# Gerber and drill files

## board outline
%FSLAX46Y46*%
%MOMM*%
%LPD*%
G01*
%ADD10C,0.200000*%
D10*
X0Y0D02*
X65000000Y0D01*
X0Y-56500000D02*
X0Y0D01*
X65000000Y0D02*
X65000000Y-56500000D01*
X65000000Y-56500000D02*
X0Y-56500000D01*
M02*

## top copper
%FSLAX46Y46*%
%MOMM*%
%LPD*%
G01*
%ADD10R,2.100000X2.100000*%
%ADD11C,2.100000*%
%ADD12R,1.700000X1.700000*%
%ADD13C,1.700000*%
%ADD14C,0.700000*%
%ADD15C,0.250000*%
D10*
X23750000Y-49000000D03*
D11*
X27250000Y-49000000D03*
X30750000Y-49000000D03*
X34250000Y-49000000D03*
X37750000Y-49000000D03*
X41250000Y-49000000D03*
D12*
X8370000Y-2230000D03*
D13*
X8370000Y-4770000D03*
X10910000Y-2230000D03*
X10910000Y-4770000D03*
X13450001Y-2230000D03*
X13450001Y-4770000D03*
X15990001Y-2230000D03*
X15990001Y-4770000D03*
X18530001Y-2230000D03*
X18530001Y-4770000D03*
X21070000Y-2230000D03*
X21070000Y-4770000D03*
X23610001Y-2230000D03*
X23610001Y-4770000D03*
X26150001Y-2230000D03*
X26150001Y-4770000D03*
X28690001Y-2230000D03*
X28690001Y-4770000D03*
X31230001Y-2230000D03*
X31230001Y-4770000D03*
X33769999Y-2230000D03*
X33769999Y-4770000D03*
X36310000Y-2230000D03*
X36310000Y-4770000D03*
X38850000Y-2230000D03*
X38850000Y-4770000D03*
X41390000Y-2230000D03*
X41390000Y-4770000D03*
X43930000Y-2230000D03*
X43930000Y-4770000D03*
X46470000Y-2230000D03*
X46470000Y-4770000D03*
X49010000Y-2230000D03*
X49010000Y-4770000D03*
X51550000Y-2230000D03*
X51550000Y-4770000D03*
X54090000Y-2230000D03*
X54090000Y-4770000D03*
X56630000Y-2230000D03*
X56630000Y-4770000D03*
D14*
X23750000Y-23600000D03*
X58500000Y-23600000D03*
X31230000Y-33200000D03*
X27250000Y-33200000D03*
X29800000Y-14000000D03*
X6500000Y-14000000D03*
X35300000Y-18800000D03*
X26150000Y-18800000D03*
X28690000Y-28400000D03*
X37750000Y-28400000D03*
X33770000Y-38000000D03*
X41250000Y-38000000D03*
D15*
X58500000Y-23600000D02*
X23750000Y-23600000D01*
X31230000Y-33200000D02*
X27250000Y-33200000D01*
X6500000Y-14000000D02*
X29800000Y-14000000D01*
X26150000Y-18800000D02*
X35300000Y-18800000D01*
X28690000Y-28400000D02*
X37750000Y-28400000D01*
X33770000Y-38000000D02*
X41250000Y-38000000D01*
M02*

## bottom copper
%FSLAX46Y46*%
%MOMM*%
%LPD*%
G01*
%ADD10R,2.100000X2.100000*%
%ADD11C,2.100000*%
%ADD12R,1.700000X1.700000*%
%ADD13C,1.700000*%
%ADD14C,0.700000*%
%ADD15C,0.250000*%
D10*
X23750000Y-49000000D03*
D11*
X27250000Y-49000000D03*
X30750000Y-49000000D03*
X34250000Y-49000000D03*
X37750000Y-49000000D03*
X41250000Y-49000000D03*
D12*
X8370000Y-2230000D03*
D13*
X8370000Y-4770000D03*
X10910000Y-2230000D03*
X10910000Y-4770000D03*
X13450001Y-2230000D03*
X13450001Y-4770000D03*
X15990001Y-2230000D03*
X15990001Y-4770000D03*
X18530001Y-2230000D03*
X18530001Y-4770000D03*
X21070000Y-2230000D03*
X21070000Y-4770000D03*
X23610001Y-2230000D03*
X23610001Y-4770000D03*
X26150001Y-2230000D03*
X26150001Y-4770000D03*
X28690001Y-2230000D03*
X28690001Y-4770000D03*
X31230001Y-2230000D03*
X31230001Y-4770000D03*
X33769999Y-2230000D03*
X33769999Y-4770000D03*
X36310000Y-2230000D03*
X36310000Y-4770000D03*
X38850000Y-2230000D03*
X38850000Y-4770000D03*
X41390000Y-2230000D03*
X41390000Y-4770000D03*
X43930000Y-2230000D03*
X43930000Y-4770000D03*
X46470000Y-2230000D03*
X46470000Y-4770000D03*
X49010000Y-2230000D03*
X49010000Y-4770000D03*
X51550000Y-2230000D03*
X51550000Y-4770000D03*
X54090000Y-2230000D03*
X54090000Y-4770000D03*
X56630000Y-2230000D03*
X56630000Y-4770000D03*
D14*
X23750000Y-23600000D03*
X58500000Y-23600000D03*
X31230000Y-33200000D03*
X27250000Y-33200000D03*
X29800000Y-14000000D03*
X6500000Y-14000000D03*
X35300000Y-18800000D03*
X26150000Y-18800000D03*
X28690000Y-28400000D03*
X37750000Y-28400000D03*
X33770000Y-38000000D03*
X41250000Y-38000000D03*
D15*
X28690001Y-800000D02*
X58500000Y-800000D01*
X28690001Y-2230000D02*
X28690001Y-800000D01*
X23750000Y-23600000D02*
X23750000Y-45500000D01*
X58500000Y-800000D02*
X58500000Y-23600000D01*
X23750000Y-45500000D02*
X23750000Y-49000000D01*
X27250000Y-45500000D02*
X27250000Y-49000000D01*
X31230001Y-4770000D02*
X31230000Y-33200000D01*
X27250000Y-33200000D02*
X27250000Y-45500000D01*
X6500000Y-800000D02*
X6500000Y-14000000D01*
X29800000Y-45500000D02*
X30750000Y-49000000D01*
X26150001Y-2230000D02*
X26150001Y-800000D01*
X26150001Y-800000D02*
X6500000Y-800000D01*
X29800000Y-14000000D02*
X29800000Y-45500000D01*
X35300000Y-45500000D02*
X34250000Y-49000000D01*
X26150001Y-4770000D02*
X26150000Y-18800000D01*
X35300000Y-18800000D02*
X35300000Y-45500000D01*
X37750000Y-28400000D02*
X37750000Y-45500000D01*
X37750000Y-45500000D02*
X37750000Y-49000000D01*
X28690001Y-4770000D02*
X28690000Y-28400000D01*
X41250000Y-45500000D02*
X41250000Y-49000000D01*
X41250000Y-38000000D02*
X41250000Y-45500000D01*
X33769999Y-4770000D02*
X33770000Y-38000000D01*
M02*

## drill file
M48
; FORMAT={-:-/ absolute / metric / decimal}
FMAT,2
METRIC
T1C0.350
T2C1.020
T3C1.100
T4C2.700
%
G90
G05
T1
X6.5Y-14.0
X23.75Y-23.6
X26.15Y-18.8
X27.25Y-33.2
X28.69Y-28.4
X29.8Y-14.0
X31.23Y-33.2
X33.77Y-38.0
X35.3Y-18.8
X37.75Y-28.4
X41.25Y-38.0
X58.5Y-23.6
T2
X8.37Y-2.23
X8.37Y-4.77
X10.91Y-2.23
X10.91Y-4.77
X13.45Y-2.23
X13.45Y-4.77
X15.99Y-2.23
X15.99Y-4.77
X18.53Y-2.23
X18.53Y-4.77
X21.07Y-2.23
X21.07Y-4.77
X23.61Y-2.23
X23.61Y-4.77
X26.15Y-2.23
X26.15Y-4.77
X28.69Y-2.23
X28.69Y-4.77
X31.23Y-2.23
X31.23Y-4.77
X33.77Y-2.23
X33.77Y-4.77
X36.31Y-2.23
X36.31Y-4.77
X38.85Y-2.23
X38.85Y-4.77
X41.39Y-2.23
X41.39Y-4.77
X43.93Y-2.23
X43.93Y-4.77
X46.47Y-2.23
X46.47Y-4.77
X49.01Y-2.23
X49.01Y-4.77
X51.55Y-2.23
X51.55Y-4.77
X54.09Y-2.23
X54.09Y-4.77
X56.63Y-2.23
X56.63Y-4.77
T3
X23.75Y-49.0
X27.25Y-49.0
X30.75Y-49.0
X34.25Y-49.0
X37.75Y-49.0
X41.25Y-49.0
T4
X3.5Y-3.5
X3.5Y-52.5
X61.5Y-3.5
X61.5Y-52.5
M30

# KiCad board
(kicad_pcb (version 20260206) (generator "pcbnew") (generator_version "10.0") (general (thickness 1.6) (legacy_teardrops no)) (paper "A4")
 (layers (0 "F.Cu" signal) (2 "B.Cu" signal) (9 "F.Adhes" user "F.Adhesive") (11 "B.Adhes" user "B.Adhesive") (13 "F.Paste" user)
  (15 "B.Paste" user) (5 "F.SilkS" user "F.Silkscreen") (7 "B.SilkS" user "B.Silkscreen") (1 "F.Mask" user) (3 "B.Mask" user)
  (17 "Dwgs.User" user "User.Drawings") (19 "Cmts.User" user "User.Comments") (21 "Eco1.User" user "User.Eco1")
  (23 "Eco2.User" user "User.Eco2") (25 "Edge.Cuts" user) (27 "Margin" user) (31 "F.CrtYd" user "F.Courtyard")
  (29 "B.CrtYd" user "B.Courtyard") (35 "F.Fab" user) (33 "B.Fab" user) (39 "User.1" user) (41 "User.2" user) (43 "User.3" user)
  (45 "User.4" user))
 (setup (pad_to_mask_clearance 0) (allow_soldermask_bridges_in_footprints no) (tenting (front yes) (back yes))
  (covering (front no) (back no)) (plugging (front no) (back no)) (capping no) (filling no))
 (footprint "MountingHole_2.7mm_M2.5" (layer "F.Cu") (at 61.5 52.5)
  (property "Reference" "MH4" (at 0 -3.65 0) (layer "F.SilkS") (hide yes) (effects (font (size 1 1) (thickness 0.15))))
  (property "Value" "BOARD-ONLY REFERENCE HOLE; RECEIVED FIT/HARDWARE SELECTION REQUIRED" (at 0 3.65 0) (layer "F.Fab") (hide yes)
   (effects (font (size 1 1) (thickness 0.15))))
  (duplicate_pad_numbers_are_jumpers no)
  (pad "" np_thru_hole circle (at 0 0) (size 2.7 2.7) (drill 2.7) (layers "*.Cu")))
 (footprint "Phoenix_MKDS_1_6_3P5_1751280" (layer "F.Cu") (at 32.5 49)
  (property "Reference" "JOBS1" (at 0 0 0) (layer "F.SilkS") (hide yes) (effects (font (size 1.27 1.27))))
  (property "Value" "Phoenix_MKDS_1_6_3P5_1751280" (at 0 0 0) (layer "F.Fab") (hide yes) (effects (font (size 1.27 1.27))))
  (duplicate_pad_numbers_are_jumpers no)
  (pad "1" thru_hole rect (at -8.75 0) (size 2.1 2.1) (drill 1.1) (layers "*.Cu") (remove_unused_layers no) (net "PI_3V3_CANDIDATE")
   (thermal_bridge_angle 45))
  (pad "2" thru_hole circle (at -5.25 0) (size 2.1 2.1) (drill 1.1) (layers "*.Cu") (remove_unused_layers no) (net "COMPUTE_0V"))
  (pad "3" thru_hole circle (at -1.75 0) (size 2.1 2.1) (drill 1.1) (layers "*.Cu") (remove_unused_layers no) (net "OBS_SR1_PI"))
  (pad "4" thru_hole circle (at 1.75 0) (size 2.1 2.1) (drill 1.1) (layers "*.Cu") (remove_unused_layers no) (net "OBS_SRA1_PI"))
  (pad "5" thru_hole circle (at 5.25 0) (size 2.1 2.1) (drill 1.1) (layers "*.Cu") (remove_unused_layers no) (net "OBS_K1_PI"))
  (pad "6" thru_hole circle (at 8.75 0) (size 2.1 2.1) (drill 1.1) (layers "*.Cu") (remove_unused_layers no) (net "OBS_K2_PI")))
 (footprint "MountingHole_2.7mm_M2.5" (layer "F.Cu") (at 3.5 3.5)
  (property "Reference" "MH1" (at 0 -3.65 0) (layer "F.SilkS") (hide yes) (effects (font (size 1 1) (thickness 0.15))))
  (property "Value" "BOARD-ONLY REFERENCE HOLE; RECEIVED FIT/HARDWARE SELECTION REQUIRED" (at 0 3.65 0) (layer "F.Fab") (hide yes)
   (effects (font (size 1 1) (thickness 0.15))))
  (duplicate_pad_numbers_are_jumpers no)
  (pad "" np_thru_hole circle (at 0 0) (size 2.7 2.7) (drill 2.7) (layers "*.Cu")))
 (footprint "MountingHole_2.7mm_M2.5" (layer "F.Cu") (at 61.5 3.5)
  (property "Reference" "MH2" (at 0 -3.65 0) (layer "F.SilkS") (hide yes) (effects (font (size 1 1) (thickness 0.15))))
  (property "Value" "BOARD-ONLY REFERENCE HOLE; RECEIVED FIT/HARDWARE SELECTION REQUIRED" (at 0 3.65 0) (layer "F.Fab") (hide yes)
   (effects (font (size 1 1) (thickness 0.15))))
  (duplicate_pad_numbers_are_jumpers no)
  (pad "" np_thru_hole circle (at 0 0) (size 2.7 2.7) (drill 2.7) (layers "*.Cu")))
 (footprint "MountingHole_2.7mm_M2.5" (layer "F.Cu") (at 3.5 52.5)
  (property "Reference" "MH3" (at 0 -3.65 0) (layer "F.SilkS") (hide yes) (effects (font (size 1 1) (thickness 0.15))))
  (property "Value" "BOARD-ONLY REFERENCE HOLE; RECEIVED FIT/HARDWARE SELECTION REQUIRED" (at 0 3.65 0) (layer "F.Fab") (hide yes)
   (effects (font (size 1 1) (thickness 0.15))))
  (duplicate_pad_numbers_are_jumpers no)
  (pad "" np_thru_hole circle (at 0 0) (size 2.7 2.7) (drill 2.7) (layers "*.Cu")))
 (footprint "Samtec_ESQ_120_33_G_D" (layer "F.Cu") (at 32.5 3.5)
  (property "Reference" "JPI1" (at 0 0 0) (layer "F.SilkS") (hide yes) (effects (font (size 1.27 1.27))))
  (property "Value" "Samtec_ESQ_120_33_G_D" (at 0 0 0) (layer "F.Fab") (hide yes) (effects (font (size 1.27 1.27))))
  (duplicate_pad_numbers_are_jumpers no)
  (pad "1" thru_hole rect (at -24.13 -1.27) (size 1.7 1.7) (drill 1.02) (layers "*.Cu") (remove_unused_layers no) (thermal_bridge_angle 45))
  (pad "2" thru_hole circle (at -24.13 1.27) (size 1.7 1.7) (drill 1.02) (layers "*.Cu") (remove_unused_layers no))
  (pad "3" thru_hole circle (at -21.59 -1.27) (size 1.7 1.7) (drill 1.02) (layers "*.Cu") (remove_unused_layers no))
  (pad "4" thru_hole circle (at -21.59 1.27) (size 1.7 1.7) (drill 1.02) (layers "*.Cu") (remove_unused_layers no))
  (pad "5" thru_hole circle (at -19.049999 -1.27) (size 1.7 1.7) (drill 1.02) (layers "*.Cu") (remove_unused_layers no))
  (pad "6" thru_hole circle (at -19.049999 1.27) (size 1.7 1.7) (drill 1.02) (layers "*.Cu") (remove_unused_layers no))
  (pad "7" thru_hole circle (at -16.509999 -1.27) (size 1.7 1.7) (drill 1.02) (layers "*.Cu") (remove_unused_layers no))
  (pad "8" thru_hole circle (at -16.509999 1.27) (size 1.7 1.7) (drill 1.02) (layers "*.Cu") (remove_unused_layers no))
  (pad "9" thru_hole circle (at -13.969999 -1.27) (size 1.7 1.7) (drill 1.02) (layers "*.Cu") (remove_unused_layers no))
  (pad "10" thru_hole circle (at -13.969999 1.27) (size 1.7 1.7) (drill 1.02) (layers "*.Cu") (remove_unused_layers no))
  (pad "11" thru_hole circle (at -11.43 -1.27) (size 1.7 1.7) (drill 1.02) (layers "*.Cu") (remove_unused_layers no))
  (pad "12" thru_hole circle (at -11.43 1.27) (size 1.7 1.7) (drill 1.02) (layers "*.Cu") (remove_unused_layers no))
  (pad "13" thru_hole circle (at -8.889999 -1.27) (size 1.7 1.7) (drill 1.02) (layers "*.Cu") (remove_unused_layers no))
  (pad "14" thru_hole circle (at -8.889999 1.27) (size 1.7 1.7) (drill 1.02) (layers "*.Cu") (remove_unused_layers no))
  (pad "15" thru_hole circle (at -6.349999 -1.27) (size 1.7 1.7) (drill 1.02) (layers "*.Cu") (remove_unused_layers no) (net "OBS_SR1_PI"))
  (pad "16" thru_hole circle (at -6.349999 1.27) (size 1.7 1.7) (drill 1.02) (layers "*.Cu") (remove_unused_layers no) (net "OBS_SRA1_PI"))
  (pad "17" thru_hole circle (at -3.809999 -1.27) (size 1.7 1.7) (drill 1.02) (layers "*.Cu") (remove_unused_layers no)
   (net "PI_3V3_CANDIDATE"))
  (pad "18" thru_hole circle (at -3.809999 1.27) (size 1.7 1.7) (drill 1.02) (layers "*.Cu") (remove_unused_layers no) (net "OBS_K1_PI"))
  (pad "19" thru_hole circle (at -1.269999 -1.27) (size 1.7 1.7) (drill 1.02) (layers "*.Cu") (remove_unused_layers no))
  (pad "20" thru_hole circle (at -1.269999 1.27) (size 1.7 1.7) (drill 1.02) (layers "*.Cu") (remove_unused_layers no) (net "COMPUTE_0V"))
  (pad "21" thru_hole circle (at 1.269999 -1.27) (size 1.7 1.7) (drill 1.02) (layers "*.Cu") (remove_unused_layers no))
  (pad "22" thru_hole circle (at 1.269999 1.27) (size 1.7 1.7) (drill 1.02) (layers "*.Cu") (remove_unused_layers no) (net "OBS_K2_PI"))
  (pad "23" thru_hole circle (at 3.81 -1.27) (size 1.7 1.7) (drill 1.02) (layers "*.Cu") (remove_unused_layers no))
  (pad "24" thru_hole circle (at 3.81 1.27) (size 1.7 1.7) (drill 1.02) (layers "*.Cu") (remove_unused_layers no))
  (pad "25" thru_hole circle (at 6.35 -1.27) (size 1.7 1.7) (drill 1.02) (layers "*.Cu") (remove_unused_layers no))
  (pad "26" thru_hole circle (at 6.35 1.27) (size 1.7 1.7) (drill 1.02) (layers "*.Cu") (remove_unused_layers no))
  (pad "27" thru_hole circle (at 8.89 -1.27) (size 1.7 1.7) (drill 1.02) (layers "*.Cu") (remove_unused_layers no))
  (pad "28" thru_hole circle (at 8.89 1.27) (size 1.7 1.7) (drill 1.02) (layers "*.Cu") (remove_unused_layers no))
  (pad "29" thru_hole circle (at 11.43 -1.27) (size 1.7 1.7) (drill 1.02) (layers "*.Cu") (remove_unused_layers no))
  (pad "30" thru_hole circle (at 11.43 1.27) (size 1.7 1.7) (drill 1.02) (layers "*.Cu") (remove_unused_layers no))
  (pad "31" thru_hole circle (at 13.97 -1.27) (size 1.7 1.7) (drill 1.02) (layers "*.Cu") (remove_unused_layers no))
  (pad "32" thru_hole circle (at 13.97 1.27) (size 1.7 1.7) (drill 1.02) (layers "*.Cu") (remove_unused_layers no))
  (pad "33" thru_hole circle (at 16.51 -1.27) (size 1.7 1.7) (drill 1.02) (layers "*.Cu") (remove_unused_layers no))
  (pad "34" thru_hole circle (at 16.51 1.27) (size 1.7 1.7) (drill 1.02) (layers "*.Cu") (remove_unused_layers no))
  (pad "35" thru_hole circle (at 19.05 -1.27) (size 1.7 1.7) (drill 1.02) (layers "*.Cu") (remove_unused_layers no))
  (pad "36" thru_hole circle (at 19.05 1.27) (size 1.7 1.7) (drill 1.02) (layers "*.Cu") (remove_unused_layers no))
  (pad "37" thru_hole circle (at 21.59 -1.27) (size 1.7 1.7) (drill 1.02) (layers "*.Cu") (remove_unused_layers no))
  (pad "38" thru_hole circle (at 21.59 1.27) (size 1.7 1.7) (drill 1.02) (layers "*.Cu") (remove_unused_layers no))
  (pad "39" thru_hole circle (at 24.13 -1.27) (size 1.7 1.7) (drill 1.02) (layers "*.Cu") (remove_unused_layers no))
  (pad "40" thru_hole circle (at 24.13 1.27) (size 1.7 1.7) (drill 1.02) (layers "*.Cu") (remove_unused_layers no)))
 (gr_line (start 0 0) (end 65 0) (stroke (width 0.2) (type default)) (layer "Edge.Cuts"))
 (gr_line (start 0 56.5) (end 0 0) (stroke (width 0.2) (type default)) (layer "Edge.Cuts"))
 (gr_line (start 65 0) (end 65 56.5) (stroke (width 0.2) (type default)) (layer "Edge.Cuts"))
 (gr_line (start 65 56.5) (end 0 56.5) (stroke (width 0.2) (type default)) (layer "Edge.Cuts"))
 (segment (start 58.5 23.6) (end 23.75 23.6) (width 0.25) (layer "F.Cu") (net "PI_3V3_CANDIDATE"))
 (via (at 23.75 23.6) (size 0.7) (drill 0.35) (layers "F.Cu" "B.Cu") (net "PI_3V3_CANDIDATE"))
 (via (at 58.5 23.6) (size 0.7) (drill 0.35) (layers "F.Cu" "B.Cu") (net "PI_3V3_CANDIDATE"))
 (segment (start 28.690001 0.8) (end 58.5 0.8) (width 0.25) (layer "B.Cu") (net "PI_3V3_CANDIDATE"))
 (segment (start 28.690001 2.23) (end 28.690001 0.8) (width 0.25) (layer "B.Cu") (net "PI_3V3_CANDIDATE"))
 (segment (start 23.75 23.6) (end 23.75 45.5) (width 0.25) (layer "B.Cu") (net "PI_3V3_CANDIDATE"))
 (segment (start 58.5 0.8) (end 58.5 23.6) (width 0.25) (layer "B.Cu") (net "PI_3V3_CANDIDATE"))
 (segment (start 23.75 45.5) (end 23.75 49) (width 0.25) (layer "B.Cu") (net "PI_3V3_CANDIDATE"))
 (segment (start 31.23 33.2) (end 27.25 33.2) (width 0.25) (layer "F.Cu") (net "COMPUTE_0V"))
 (via (at 31.23 33.2) (size 0.7) (drill 0.35) (layers "F.Cu" "B.Cu") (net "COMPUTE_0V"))
 (via (at 27.25 33.2) (size 0.7) (drill 0.35) (layers "F.Cu" "B.Cu") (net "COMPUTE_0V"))
 (segment (start 27.25 45.5) (end 27.25 49) (width 0.25) (layer "B.Cu") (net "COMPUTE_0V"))
 (segment (start 31.230001 4.77) (end 31.23 33.2) (width 0.25) (layer "B.Cu") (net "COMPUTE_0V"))
 (segment (start 27.25 33.2) (end 27.25 45.5) (width 0.25) (layer "B.Cu") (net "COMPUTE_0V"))
 (segment (start 6.5 14) (end 29.8 14) (width 0.25) (layer "F.Cu") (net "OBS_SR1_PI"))
 (via (at 29.8 14) (size 0.7) (drill 0.35) (layers "F.Cu" "B.Cu") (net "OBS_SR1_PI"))
 (via (at 6.5 14) (size 0.7) (drill 0.35) (layers "F.Cu" "B.Cu") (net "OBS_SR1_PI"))
 (segment (start 6.5 0.8) (end 6.5 14) (width 0.25) (layer "B.Cu") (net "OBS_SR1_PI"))
 (segment (start 29.8 45.5) (end 30.75 49) (width 0.25) (layer "B.Cu") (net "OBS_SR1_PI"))
 (segment (start 26.150001 2.23) (end 26.150001 0.8) (width 0.25) (layer "B.Cu") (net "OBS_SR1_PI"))
 (segment (start 26.150001 0.8) (end 6.5 0.8) (width 0.25) (layer "B.Cu") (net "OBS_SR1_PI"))
 (segment (start 29.8 14) (end 29.8 45.5) (width 0.25) (layer "B.Cu") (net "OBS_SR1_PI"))
 (segment (start 26.15 18.8) (end 35.3 18.8) (width 0.25) (layer "F.Cu") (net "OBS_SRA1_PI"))
 (via (at 35.3 18.8) (size 0.7) (drill 0.35) (layers "F.Cu" "B.Cu") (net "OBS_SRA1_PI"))
 (via (at 26.15 18.8) (size 0.7) (drill 0.35) (layers "F.Cu" "B.Cu") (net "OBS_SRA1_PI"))
 (segment (start 35.3 45.5) (end 34.25 49) (width 0.25) (layer "B.Cu") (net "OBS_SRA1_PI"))
 (segment (start 26.150001 4.77) (end 26.15 18.8) (width 0.25) (layer "B.Cu") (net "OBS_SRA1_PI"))
 (segment (start 35.3 18.8) (end 35.3 45.5) (width 0.25) (layer "B.Cu") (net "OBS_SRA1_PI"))
 (segment (start 28.69 28.4) (end 37.75 28.4) (width 0.25) (layer "F.Cu") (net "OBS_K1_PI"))
 (via (at 28.69 28.4) (size 0.7) (drill 0.35) (layers "F.Cu" "B.Cu") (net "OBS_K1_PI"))
 (via (at 37.75 28.4) (size 0.7) (drill 0.35) (layers "F.Cu" "B.Cu") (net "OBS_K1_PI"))
 (segment (start 37.75 28.4) (end 37.75 45.5) (width 0.25) (layer "B.Cu") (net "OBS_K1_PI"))
 (segment (start 37.75 45.5) (end 37.75 49) (width 0.25) (layer "B.Cu") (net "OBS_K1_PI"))
 (segment (start 28.690001 4.77) (end 28.69 28.4) (width 0.25) (layer "B.Cu") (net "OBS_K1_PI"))
 (segment (start 33.77 38) (end 41.25 38) (width 0.25) (layer "F.Cu") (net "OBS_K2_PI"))
 (via (at 33.77 38) (size 0.7) (drill 0.35) (layers "F.Cu" "B.Cu") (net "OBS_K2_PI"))
 (via (at 41.25 38) (size 0.7) (drill 0.35) (layers "F.Cu" "B.Cu") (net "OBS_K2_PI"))
 (segment (start 41.25 45.5) (end 41.25 49) (width 0.25) (layer "B.Cu") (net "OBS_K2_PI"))
 (segment (start 41.25 38) (end 41.25 45.5) (width 0.25) (layer "B.Cu") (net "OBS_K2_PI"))
 (segment (start 33.769999 4.77) (end 33.77 38) (width 0.25) (layer "B.Cu") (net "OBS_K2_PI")))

